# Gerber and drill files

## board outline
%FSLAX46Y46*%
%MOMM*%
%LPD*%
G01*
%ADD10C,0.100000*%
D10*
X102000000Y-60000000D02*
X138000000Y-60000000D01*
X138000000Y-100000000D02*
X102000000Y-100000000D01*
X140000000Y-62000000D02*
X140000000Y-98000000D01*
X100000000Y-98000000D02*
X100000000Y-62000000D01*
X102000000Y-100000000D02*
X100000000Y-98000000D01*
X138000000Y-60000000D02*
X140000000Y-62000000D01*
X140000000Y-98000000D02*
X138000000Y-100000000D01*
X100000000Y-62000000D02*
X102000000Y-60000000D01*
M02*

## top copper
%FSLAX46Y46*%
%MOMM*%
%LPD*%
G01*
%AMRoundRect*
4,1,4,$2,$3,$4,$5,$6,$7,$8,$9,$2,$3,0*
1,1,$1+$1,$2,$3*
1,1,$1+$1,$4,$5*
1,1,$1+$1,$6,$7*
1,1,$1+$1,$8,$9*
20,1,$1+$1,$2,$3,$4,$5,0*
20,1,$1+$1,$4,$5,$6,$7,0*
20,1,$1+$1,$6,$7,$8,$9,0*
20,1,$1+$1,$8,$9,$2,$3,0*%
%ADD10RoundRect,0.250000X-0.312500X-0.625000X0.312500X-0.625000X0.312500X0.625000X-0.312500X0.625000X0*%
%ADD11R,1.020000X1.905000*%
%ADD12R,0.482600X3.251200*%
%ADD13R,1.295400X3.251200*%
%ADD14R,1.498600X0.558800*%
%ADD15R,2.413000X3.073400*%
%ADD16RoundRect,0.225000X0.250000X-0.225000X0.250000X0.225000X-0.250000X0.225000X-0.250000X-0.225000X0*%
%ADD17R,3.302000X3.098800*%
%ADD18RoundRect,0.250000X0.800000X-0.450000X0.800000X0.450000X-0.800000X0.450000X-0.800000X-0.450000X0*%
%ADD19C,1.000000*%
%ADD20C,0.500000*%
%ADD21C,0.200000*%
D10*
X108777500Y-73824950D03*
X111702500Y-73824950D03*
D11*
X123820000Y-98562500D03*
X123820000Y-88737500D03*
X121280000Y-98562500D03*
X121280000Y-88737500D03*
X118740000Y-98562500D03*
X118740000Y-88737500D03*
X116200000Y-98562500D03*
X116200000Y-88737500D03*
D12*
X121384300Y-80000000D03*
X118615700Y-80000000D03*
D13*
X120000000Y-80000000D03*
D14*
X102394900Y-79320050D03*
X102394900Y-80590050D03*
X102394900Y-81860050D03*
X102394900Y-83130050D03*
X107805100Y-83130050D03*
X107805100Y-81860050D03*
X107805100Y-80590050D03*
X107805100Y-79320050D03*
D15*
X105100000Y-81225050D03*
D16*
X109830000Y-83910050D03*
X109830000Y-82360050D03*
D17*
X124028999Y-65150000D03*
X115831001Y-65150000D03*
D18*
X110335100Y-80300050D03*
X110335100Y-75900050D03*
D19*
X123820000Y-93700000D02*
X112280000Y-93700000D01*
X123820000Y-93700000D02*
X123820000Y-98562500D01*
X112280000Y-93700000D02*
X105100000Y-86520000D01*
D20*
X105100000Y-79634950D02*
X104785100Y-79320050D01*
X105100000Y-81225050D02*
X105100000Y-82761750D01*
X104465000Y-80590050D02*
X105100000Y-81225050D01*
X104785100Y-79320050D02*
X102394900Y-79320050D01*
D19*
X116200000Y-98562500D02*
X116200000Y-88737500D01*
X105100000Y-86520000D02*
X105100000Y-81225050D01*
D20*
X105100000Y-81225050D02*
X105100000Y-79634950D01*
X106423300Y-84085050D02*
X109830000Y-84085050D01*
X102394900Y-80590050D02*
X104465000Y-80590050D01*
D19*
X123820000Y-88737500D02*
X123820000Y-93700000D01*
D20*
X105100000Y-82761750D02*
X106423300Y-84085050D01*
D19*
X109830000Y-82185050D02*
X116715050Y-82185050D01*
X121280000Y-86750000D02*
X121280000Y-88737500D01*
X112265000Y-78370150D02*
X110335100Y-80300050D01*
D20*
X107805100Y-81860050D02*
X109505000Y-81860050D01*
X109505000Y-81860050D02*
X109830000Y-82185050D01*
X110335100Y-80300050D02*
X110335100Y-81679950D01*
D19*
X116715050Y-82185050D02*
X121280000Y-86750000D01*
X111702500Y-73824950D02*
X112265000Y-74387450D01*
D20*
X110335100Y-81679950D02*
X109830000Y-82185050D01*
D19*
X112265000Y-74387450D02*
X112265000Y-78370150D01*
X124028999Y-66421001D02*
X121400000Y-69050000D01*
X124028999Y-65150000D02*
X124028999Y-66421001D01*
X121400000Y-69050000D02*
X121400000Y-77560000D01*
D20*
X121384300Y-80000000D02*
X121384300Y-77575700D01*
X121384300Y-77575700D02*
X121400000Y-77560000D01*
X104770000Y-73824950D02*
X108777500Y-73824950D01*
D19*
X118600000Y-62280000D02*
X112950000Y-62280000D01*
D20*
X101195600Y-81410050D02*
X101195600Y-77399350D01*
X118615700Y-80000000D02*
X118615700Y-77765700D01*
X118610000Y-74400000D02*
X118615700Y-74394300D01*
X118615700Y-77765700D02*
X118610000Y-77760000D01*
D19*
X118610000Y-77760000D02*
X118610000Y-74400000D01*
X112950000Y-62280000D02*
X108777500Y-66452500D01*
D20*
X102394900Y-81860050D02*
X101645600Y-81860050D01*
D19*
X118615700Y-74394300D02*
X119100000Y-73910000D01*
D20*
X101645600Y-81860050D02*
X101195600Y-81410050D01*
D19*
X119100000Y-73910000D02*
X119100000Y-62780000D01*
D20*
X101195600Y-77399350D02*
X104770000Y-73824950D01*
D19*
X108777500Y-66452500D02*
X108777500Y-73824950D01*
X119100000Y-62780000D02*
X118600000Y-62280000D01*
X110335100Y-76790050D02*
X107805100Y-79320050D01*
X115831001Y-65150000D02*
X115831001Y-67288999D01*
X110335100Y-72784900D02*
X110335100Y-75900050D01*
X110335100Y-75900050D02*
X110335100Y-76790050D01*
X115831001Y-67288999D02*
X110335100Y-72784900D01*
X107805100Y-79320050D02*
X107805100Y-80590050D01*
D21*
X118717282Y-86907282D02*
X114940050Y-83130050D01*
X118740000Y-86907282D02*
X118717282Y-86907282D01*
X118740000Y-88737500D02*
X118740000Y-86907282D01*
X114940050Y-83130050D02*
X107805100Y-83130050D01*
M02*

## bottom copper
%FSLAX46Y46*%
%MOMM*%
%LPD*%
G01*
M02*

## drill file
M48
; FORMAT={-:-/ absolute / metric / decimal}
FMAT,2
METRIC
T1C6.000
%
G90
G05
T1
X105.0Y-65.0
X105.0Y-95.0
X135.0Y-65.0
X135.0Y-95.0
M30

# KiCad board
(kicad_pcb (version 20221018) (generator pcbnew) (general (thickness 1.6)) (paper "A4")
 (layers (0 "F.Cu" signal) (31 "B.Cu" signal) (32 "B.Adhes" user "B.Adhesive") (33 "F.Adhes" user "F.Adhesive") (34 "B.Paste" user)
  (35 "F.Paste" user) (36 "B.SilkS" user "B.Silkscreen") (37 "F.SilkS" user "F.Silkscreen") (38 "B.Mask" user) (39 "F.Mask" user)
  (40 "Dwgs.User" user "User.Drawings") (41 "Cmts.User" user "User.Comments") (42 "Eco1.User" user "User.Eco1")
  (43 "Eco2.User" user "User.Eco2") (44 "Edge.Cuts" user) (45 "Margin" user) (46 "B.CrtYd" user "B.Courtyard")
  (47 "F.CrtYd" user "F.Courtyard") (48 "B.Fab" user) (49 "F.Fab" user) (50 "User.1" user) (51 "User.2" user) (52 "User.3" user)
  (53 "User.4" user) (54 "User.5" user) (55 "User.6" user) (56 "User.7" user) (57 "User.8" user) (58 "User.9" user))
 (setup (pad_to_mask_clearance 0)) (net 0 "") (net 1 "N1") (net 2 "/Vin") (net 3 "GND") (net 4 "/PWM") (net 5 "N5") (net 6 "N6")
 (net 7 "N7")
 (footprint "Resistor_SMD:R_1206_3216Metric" (layer "F.Cu") (at 110.24 73.82495)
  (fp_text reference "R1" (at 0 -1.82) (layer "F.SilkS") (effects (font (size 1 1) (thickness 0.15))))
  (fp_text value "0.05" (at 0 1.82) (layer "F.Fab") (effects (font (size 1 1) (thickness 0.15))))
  (pad "1" smd roundrect (at -1.4625 0) (size 1.125 1.75) (layers "F.Cu" "F.Paste" "F.Mask") (roundrect_rratio 0.222222) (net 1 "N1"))
  (pad "2" smd roundrect (at 1.4625 0) (size 1.125 1.75) (layers "F.Cu" "F.Paste" "F.Mask") (roundrect_rratio 0.222222) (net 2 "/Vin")))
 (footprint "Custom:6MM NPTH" (layer "F.Cu") (at 135 95)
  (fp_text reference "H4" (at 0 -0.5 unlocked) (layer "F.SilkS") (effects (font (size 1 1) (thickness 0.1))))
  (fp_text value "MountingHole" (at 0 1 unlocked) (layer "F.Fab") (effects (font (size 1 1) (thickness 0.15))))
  (pad "" np_thru_hole circle (at 0 0) (size 6 6) (drill 6) (layers "F&B.Cu" "*.Mask")))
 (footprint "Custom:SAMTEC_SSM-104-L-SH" (layer "F.Cu") (at 120.01 93.65 180)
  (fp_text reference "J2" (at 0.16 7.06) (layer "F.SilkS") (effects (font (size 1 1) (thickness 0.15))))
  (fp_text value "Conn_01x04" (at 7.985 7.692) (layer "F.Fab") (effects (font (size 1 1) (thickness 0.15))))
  (pad "1" smd rect (at -3.81 -4.9125 180) (size 1.02 1.905) (layers "F.Cu" "F.Paste" "F.Mask") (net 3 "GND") (solder_mask_margin 0.102))
  (pad "1" smd rect (at -3.81 4.9125 180) (size 1.02 1.905) (layers "F.Cu" "F.Paste" "F.Mask") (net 3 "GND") (solder_mask_margin 0.102))
  (pad "2" smd rect (at -1.27 -4.9125 180) (size 1.02 1.905) (layers "F.Cu" "F.Paste" "F.Mask") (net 2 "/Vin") (solder_mask_margin 0.102))
  (pad "2" smd rect (at -1.27 4.9125 180) (size 1.02 1.905) (layers "F.Cu" "F.Paste" "F.Mask") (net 2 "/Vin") (solder_mask_margin 0.102))
  (pad "3" smd rect (at 1.27 -4.9125 180) (size 1.02 1.905) (layers "F.Cu" "F.Paste" "F.Mask") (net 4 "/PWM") (solder_mask_margin 0.102))
  (pad "3" smd rect (at 1.27 4.9125 180) (size 1.02 1.905) (layers "F.Cu" "F.Paste" "F.Mask") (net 4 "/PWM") (solder_mask_margin 0.102))
  (pad "4" smd rect (at 3.81 -4.9125 180) (size 1.02 1.905) (layers "F.Cu" "F.Paste" "F.Mask") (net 3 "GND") (solder_mask_margin 0.102))
  (pad "4" smd rect (at 3.81 4.9125 180) (size 1.02 1.905) (layers "F.Cu" "F.Paste" "F.Mask") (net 3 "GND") (solder_mask_margin 0.102)))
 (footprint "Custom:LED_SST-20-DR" (layer "F.Cu") (at 120 80 180)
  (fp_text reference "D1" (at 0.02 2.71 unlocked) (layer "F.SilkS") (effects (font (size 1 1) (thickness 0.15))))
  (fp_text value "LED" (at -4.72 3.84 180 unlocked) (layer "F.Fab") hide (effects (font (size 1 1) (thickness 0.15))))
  (pad "1" smd rect (at -1.3843 0 180) (size 0.4826 3.2512) (layers "F.Cu" "F.Paste" "F.Mask") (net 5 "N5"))
  (pad "2" smd rect (at 1.3843 0 180) (size 0.4826 3.2512) (layers "F.Cu" "F.Paste" "F.Mask") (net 1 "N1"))
  (pad "3" smd rect (at 0 0 180) (size 1.2954 3.2512) (layers "F.Cu" "F.Paste" "F.Mask")))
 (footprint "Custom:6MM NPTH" (layer "F.Cu") (at 105 65)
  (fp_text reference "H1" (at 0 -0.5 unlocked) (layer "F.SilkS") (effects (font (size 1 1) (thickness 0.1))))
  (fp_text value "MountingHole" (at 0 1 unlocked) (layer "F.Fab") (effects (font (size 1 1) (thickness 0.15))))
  (pad "" np_thru_hole circle (at 0 0) (size 6 6) (drill 6) (layers "F&B.Cu" "*.Mask")))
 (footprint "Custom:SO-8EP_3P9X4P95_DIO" (layer "F.Cu") (at 105.1 81.22505)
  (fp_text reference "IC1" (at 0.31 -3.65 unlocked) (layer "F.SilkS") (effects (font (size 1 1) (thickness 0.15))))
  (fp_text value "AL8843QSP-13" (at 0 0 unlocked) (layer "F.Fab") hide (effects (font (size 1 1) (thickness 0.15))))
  (pad "1" smd rect (at -2.7051 -1.905) (size 1.4986 0.5588) (layers "F.Cu" "F.Paste" "F.Mask") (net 3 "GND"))
  (pad "2" smd rect (at -2.7051 -0.635) (size 1.4986 0.5588) (layers "F.Cu" "F.Paste" "F.Mask") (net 3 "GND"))
  (pad "3" smd rect (at -2.7051 0.635) (size 1.4986 0.5588) (layers "F.Cu" "F.Paste" "F.Mask") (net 1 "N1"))
  (pad "4" smd rect (at -2.7051 1.905) (size 1.4986 0.5588) (layers "F.Cu" "F.Paste" "F.Mask") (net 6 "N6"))
  (pad "5" smd rect (at 2.7051 1.905) (size 1.4986 0.5588) (layers "F.Cu" "F.Paste" "F.Mask") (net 4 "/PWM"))
  (pad "6" smd rect (at 2.7051 0.635) (size 1.4986 0.5588) (layers "F.Cu" "F.Paste" "F.Mask") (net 2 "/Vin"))
  (pad "7" smd rect (at 2.7051 -0.635) (size 1.4986 0.5588) (layers "F.Cu" "F.Paste" "F.Mask") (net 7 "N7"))
  (pad "8" smd rect (at 2.7051 -1.905) (size 1.4986 0.5588) (layers "F.Cu" "F.Paste" "F.Mask") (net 7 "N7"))
  (pad "EPAD" smd rect (at 0 0) (size 2.413 3.0734) (layers "F.Cu" "F.Mask") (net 3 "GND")))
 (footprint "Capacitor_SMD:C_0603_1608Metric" (layer "F.Cu") (at 109.83 83.13505 90)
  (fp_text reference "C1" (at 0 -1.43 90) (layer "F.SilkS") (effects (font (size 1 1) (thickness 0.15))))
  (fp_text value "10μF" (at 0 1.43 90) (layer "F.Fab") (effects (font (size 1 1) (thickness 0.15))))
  (pad "1" smd roundrect (at -0.775 0 90) (size 0.9 0.95) (layers "F.Cu" "F.Paste" "F.Mask") (roundrect_rratio 0.25) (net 3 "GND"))
  (pad "2" smd roundrect (at 0.775 0 90) (size 0.9 0.95) (layers "F.Cu" "F.Paste" "F.Mask") (roundrect_rratio 0.25) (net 2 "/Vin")))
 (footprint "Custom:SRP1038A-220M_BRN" (layer "F.Cu") (at 119.93 65.15 180)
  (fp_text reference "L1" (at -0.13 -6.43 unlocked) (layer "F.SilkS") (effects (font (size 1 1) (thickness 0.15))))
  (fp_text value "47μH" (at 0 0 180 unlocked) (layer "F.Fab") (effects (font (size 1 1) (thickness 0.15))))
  (pad "1" smd rect (at -4.098999 0 180) (size 3.302 3.0988) (layers "F.Cu" "F.Paste" "F.Mask") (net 5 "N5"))
  (pad "2" smd rect (at 4.098999 0 180) (size 3.302 3.0988) (layers "F.Cu" "F.Paste" "F.Mask") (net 7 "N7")))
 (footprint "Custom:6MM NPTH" (layer "F.Cu") (at 105 95)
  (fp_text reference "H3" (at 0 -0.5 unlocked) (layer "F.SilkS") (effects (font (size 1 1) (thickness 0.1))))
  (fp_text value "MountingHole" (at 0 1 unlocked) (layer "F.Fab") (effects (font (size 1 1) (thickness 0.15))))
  (pad "" np_thru_hole circle (at 0 0) (size 6 6) (drill 6) (layers "F&B.Cu" "*.Mask")))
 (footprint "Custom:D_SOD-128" (layer "F.Cu") (at 110.3351 78.10005 90)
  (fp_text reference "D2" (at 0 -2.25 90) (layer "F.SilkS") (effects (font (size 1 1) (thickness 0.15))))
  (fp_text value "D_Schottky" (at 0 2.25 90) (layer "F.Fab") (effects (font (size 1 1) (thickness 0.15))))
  (pad "1" smd roundrect (at -2.2 0 90) (size 1.4 2.1) (layers "F.Cu" "F.Paste" "F.Mask") (roundrect_rratio 0.1785714286) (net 2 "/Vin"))
  (pad "2" smd roundrect (at 2.2 0 90) (size 1.4 2.1) (layers "F.Cu" "F.Paste" "F.Mask") (roundrect_rratio 0.1785714286) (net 7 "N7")))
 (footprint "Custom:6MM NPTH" (layer "F.Cu") (at 135 65)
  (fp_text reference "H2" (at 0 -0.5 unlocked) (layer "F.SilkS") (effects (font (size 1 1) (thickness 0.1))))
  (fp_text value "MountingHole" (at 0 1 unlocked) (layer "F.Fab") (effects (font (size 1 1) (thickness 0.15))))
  (pad "" np_thru_hole circle (at 0 0) (size 6 6) (drill 6) (layers "F&B.Cu" "*.Mask")))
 (gr_line (start 102 60) (end 138 60) (stroke (width 0.1) (type default)) (layer "Edge.Cuts"))
 (gr_line (start 138 100) (end 102 100) (stroke (width 0.1) (type default)) (layer "Edge.Cuts"))
 (gr_line (start 140 62) (end 140 98) (stroke (width 0.1) (type default)) (layer "Edge.Cuts"))
 (gr_line (start 100 98) (end 100 62) (stroke (width 0.1) (type default)) (layer "Edge.Cuts"))
 (gr_line (start 102 100) (end 100 98) (stroke (width 0.1) (type default)) (layer "Edge.Cuts"))
 (gr_line (start 138 60) (end 140 62) (stroke (width 0.1) (type default)) (layer "Edge.Cuts"))
 (gr_line (start 140 98) (end 138 100) (stroke (width 0.1) (type default)) (layer "Edge.Cuts"))
 (gr_line (start 100 62) (end 102 60) (stroke (width 0.1) (type default)) (layer "Edge.Cuts"))
 (segment (start 123.82 93.7) (end 112.28 93.7) (width 1) (layer "F.Cu") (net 3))
 (segment (start 123.82 93.7) (end 123.82 98.5625) (width 1) (layer "F.Cu") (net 3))
 (segment (start 112.28 93.7) (end 105.1 86.52) (width 1) (layer "F.Cu") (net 3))
 (segment (start 105.1 79.63495) (end 104.7851 79.32005) (width 0.5) (layer "F.Cu") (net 3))
 (segment (start 105.1 81.22505) (end 105.1 82.76175) (width 0.5) (layer "F.Cu") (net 3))
 (segment (start 104.465 80.59005) (end 105.1 81.22505) (width 0.5) (layer "F.Cu") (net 3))
 (segment (start 104.7851 79.32005) (end 102.3949 79.32005) (width 0.5) (layer "F.Cu") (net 3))
 (segment (start 116.2 98.5625) (end 116.2 88.7375) (width 1) (layer "F.Cu") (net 3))
 (segment (start 105.1 86.52) (end 105.1 81.22505) (width 1) (layer "F.Cu") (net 3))
 (segment (start 105.1 81.22505) (end 105.1 79.63495) (width 0.5) (layer "F.Cu") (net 3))
 (segment (start 106.4233 84.08505) (end 109.83 84.08505) (width 0.5) (layer "F.Cu") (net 3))
 (segment (start 102.3949 80.59005) (end 104.465 80.59005) (width 0.5) (layer "F.Cu") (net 3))
 (segment (start 123.82 88.7375) (end 123.82 93.7) (width 1) (layer "F.Cu") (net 3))
 (segment (start 105.1 82.76175) (end 106.4233 84.08505) (width 0.5) (layer "F.Cu") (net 3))
 (segment (start 109.83 82.18505) (end 116.71505 82.18505) (width 1) (layer "F.Cu") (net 2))
 (segment (start 121.28 86.75) (end 121.28 88.7375) (width 1) (layer "F.Cu") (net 2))
 (segment (start 112.265 78.37015) (end 110.3351 80.30005) (width 1) (layer "F.Cu") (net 2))
 (segment (start 107.8051 81.86005) (end 109.505 81.86005) (width 0.5) (layer "F.Cu") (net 2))
 (segment (start 109.505 81.86005) (end 109.83 82.18505) (width 0.5) (layer "F.Cu") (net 2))
 (segment (start 110.3351 80.30005) (end 110.3351 81.67995) (width 0.5) (layer "F.Cu") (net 2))
 (segment (start 116.71505 82.18505) (end 121.28 86.75) (width 1) (layer "F.Cu") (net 2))
 (segment (start 111.7025 73.82495) (end 112.265 74.38745) (width 1) (layer "F.Cu") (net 2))
 (segment (start 110.3351 81.67995) (end 109.83 82.18505) (width 0.5) (layer "F.Cu") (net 2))
 (segment (start 112.265 74.38745) (end 112.265 78.37015) (width 1) (layer "F.Cu") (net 2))
 (segment (start 124.028999 66.421001) (end 121.4 69.05) (width 1) (layer "F.Cu") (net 5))
 (segment (start 124.028999 65.15) (end 124.028999 66.421001) (width 1) (layer "F.Cu") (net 5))
 (segment (start 121.4 69.05) (end 121.4 77.56) (width 1) (layer "F.Cu") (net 5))
 (segment (start 121.3843 80) (end 121.3843 77.5757) (width 0.5) (layer "F.Cu") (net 5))
 (segment (start 121.3843 77.5757) (end 121.4 77.56) (width 0.5) (layer "F.Cu") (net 5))
 (segment (start 104.77 73.82495) (end 108.7775 73.82495) (width 0.5) (layer "F.Cu") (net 1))
 (segment (start 118.6 62.28) (end 112.95 62.28) (width 1) (layer "F.Cu") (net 1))
 (segment (start 101.1956 81.41005) (end 101.1956 77.39935) (width 0.5) (layer "F.Cu") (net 1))
 (segment (start 118.6157 80) (end 118.6157 77.7657) (width 0.5) (layer "F.Cu") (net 1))
 (segment (start 118.61 74.4) (end 118.6157 74.3943) (width 0.5) (layer "F.Cu") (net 1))
 (segment (start 118.6157 77.7657) (end 118.61 77.76) (width 0.5) (layer "F.Cu") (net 1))
 (segment (start 118.61 77.76) (end 118.61 74.4) (width 1) (layer "F.Cu") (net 1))
 (segment (start 112.95 62.28) (end 108.7775 66.4525) (width 1) (layer "F.Cu") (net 1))
 (segment (start 102.3949 81.86005) (end 101.6456 81.86005) (width 0.5) (layer "F.Cu") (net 1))
 (segment (start 118.6157 74.3943) (end 119.1 73.91) (width 1) (layer "F.Cu") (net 1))
 (segment (start 101.6456 81.86005) (end 101.1956 81.41005) (width 0.5) (layer "F.Cu") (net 1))
 (segment (start 119.1 73.91) (end 119.1 62.78) (width 1) (layer "F.Cu") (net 1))
 (segment (start 101.1956 77.39935) (end 104.77 73.82495) (width 0.5) (layer "F.Cu") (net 1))
 (segment (start 108.7775 66.4525) (end 108.7775 73.82495) (width 1) (layer "F.Cu") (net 1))
 (segment (start 119.1 62.78) (end 118.6 62.28) (width 1) (layer "F.Cu") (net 1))
 (segment (start 110.3351 76.79005) (end 107.8051 79.32005) (width 1) (layer "F.Cu") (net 7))
 (segment (start 115.831001 65.15) (end 115.831001 67.288999) (width 1) (layer "F.Cu") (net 7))
 (segment (start 110.3351 72.7849) (end 110.3351 75.90005) (width 1) (layer "F.Cu") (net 7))
 (segment (start 110.3351 75.90005) (end 110.3351 76.79005) (width 1) (layer "F.Cu") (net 7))
 (segment (start 115.831001 67.288999) (end 110.3351 72.7849) (width 1) (layer "F.Cu") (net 7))
 (segment (start 107.8051 79.32005) (end 107.8051 80.59005) (width 1) (layer "F.Cu") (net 7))
 (segment (start 118.717282 86.907282) (end 114.94005 83.13005) (width 0.2) (layer "F.Cu") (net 4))
 (segment (start 118.74 86.907282) (end 118.717282 86.907282) (width 0.2) (layer "F.Cu") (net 4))
 (segment (start 118.74 88.7375) (end 118.74 86.907282) (width 0.2) (layer "F.Cu") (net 4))
 (segment (start 114.94005 83.13005) (end 107.8051 83.13005) (width 0.2) (layer "F.Cu") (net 4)))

